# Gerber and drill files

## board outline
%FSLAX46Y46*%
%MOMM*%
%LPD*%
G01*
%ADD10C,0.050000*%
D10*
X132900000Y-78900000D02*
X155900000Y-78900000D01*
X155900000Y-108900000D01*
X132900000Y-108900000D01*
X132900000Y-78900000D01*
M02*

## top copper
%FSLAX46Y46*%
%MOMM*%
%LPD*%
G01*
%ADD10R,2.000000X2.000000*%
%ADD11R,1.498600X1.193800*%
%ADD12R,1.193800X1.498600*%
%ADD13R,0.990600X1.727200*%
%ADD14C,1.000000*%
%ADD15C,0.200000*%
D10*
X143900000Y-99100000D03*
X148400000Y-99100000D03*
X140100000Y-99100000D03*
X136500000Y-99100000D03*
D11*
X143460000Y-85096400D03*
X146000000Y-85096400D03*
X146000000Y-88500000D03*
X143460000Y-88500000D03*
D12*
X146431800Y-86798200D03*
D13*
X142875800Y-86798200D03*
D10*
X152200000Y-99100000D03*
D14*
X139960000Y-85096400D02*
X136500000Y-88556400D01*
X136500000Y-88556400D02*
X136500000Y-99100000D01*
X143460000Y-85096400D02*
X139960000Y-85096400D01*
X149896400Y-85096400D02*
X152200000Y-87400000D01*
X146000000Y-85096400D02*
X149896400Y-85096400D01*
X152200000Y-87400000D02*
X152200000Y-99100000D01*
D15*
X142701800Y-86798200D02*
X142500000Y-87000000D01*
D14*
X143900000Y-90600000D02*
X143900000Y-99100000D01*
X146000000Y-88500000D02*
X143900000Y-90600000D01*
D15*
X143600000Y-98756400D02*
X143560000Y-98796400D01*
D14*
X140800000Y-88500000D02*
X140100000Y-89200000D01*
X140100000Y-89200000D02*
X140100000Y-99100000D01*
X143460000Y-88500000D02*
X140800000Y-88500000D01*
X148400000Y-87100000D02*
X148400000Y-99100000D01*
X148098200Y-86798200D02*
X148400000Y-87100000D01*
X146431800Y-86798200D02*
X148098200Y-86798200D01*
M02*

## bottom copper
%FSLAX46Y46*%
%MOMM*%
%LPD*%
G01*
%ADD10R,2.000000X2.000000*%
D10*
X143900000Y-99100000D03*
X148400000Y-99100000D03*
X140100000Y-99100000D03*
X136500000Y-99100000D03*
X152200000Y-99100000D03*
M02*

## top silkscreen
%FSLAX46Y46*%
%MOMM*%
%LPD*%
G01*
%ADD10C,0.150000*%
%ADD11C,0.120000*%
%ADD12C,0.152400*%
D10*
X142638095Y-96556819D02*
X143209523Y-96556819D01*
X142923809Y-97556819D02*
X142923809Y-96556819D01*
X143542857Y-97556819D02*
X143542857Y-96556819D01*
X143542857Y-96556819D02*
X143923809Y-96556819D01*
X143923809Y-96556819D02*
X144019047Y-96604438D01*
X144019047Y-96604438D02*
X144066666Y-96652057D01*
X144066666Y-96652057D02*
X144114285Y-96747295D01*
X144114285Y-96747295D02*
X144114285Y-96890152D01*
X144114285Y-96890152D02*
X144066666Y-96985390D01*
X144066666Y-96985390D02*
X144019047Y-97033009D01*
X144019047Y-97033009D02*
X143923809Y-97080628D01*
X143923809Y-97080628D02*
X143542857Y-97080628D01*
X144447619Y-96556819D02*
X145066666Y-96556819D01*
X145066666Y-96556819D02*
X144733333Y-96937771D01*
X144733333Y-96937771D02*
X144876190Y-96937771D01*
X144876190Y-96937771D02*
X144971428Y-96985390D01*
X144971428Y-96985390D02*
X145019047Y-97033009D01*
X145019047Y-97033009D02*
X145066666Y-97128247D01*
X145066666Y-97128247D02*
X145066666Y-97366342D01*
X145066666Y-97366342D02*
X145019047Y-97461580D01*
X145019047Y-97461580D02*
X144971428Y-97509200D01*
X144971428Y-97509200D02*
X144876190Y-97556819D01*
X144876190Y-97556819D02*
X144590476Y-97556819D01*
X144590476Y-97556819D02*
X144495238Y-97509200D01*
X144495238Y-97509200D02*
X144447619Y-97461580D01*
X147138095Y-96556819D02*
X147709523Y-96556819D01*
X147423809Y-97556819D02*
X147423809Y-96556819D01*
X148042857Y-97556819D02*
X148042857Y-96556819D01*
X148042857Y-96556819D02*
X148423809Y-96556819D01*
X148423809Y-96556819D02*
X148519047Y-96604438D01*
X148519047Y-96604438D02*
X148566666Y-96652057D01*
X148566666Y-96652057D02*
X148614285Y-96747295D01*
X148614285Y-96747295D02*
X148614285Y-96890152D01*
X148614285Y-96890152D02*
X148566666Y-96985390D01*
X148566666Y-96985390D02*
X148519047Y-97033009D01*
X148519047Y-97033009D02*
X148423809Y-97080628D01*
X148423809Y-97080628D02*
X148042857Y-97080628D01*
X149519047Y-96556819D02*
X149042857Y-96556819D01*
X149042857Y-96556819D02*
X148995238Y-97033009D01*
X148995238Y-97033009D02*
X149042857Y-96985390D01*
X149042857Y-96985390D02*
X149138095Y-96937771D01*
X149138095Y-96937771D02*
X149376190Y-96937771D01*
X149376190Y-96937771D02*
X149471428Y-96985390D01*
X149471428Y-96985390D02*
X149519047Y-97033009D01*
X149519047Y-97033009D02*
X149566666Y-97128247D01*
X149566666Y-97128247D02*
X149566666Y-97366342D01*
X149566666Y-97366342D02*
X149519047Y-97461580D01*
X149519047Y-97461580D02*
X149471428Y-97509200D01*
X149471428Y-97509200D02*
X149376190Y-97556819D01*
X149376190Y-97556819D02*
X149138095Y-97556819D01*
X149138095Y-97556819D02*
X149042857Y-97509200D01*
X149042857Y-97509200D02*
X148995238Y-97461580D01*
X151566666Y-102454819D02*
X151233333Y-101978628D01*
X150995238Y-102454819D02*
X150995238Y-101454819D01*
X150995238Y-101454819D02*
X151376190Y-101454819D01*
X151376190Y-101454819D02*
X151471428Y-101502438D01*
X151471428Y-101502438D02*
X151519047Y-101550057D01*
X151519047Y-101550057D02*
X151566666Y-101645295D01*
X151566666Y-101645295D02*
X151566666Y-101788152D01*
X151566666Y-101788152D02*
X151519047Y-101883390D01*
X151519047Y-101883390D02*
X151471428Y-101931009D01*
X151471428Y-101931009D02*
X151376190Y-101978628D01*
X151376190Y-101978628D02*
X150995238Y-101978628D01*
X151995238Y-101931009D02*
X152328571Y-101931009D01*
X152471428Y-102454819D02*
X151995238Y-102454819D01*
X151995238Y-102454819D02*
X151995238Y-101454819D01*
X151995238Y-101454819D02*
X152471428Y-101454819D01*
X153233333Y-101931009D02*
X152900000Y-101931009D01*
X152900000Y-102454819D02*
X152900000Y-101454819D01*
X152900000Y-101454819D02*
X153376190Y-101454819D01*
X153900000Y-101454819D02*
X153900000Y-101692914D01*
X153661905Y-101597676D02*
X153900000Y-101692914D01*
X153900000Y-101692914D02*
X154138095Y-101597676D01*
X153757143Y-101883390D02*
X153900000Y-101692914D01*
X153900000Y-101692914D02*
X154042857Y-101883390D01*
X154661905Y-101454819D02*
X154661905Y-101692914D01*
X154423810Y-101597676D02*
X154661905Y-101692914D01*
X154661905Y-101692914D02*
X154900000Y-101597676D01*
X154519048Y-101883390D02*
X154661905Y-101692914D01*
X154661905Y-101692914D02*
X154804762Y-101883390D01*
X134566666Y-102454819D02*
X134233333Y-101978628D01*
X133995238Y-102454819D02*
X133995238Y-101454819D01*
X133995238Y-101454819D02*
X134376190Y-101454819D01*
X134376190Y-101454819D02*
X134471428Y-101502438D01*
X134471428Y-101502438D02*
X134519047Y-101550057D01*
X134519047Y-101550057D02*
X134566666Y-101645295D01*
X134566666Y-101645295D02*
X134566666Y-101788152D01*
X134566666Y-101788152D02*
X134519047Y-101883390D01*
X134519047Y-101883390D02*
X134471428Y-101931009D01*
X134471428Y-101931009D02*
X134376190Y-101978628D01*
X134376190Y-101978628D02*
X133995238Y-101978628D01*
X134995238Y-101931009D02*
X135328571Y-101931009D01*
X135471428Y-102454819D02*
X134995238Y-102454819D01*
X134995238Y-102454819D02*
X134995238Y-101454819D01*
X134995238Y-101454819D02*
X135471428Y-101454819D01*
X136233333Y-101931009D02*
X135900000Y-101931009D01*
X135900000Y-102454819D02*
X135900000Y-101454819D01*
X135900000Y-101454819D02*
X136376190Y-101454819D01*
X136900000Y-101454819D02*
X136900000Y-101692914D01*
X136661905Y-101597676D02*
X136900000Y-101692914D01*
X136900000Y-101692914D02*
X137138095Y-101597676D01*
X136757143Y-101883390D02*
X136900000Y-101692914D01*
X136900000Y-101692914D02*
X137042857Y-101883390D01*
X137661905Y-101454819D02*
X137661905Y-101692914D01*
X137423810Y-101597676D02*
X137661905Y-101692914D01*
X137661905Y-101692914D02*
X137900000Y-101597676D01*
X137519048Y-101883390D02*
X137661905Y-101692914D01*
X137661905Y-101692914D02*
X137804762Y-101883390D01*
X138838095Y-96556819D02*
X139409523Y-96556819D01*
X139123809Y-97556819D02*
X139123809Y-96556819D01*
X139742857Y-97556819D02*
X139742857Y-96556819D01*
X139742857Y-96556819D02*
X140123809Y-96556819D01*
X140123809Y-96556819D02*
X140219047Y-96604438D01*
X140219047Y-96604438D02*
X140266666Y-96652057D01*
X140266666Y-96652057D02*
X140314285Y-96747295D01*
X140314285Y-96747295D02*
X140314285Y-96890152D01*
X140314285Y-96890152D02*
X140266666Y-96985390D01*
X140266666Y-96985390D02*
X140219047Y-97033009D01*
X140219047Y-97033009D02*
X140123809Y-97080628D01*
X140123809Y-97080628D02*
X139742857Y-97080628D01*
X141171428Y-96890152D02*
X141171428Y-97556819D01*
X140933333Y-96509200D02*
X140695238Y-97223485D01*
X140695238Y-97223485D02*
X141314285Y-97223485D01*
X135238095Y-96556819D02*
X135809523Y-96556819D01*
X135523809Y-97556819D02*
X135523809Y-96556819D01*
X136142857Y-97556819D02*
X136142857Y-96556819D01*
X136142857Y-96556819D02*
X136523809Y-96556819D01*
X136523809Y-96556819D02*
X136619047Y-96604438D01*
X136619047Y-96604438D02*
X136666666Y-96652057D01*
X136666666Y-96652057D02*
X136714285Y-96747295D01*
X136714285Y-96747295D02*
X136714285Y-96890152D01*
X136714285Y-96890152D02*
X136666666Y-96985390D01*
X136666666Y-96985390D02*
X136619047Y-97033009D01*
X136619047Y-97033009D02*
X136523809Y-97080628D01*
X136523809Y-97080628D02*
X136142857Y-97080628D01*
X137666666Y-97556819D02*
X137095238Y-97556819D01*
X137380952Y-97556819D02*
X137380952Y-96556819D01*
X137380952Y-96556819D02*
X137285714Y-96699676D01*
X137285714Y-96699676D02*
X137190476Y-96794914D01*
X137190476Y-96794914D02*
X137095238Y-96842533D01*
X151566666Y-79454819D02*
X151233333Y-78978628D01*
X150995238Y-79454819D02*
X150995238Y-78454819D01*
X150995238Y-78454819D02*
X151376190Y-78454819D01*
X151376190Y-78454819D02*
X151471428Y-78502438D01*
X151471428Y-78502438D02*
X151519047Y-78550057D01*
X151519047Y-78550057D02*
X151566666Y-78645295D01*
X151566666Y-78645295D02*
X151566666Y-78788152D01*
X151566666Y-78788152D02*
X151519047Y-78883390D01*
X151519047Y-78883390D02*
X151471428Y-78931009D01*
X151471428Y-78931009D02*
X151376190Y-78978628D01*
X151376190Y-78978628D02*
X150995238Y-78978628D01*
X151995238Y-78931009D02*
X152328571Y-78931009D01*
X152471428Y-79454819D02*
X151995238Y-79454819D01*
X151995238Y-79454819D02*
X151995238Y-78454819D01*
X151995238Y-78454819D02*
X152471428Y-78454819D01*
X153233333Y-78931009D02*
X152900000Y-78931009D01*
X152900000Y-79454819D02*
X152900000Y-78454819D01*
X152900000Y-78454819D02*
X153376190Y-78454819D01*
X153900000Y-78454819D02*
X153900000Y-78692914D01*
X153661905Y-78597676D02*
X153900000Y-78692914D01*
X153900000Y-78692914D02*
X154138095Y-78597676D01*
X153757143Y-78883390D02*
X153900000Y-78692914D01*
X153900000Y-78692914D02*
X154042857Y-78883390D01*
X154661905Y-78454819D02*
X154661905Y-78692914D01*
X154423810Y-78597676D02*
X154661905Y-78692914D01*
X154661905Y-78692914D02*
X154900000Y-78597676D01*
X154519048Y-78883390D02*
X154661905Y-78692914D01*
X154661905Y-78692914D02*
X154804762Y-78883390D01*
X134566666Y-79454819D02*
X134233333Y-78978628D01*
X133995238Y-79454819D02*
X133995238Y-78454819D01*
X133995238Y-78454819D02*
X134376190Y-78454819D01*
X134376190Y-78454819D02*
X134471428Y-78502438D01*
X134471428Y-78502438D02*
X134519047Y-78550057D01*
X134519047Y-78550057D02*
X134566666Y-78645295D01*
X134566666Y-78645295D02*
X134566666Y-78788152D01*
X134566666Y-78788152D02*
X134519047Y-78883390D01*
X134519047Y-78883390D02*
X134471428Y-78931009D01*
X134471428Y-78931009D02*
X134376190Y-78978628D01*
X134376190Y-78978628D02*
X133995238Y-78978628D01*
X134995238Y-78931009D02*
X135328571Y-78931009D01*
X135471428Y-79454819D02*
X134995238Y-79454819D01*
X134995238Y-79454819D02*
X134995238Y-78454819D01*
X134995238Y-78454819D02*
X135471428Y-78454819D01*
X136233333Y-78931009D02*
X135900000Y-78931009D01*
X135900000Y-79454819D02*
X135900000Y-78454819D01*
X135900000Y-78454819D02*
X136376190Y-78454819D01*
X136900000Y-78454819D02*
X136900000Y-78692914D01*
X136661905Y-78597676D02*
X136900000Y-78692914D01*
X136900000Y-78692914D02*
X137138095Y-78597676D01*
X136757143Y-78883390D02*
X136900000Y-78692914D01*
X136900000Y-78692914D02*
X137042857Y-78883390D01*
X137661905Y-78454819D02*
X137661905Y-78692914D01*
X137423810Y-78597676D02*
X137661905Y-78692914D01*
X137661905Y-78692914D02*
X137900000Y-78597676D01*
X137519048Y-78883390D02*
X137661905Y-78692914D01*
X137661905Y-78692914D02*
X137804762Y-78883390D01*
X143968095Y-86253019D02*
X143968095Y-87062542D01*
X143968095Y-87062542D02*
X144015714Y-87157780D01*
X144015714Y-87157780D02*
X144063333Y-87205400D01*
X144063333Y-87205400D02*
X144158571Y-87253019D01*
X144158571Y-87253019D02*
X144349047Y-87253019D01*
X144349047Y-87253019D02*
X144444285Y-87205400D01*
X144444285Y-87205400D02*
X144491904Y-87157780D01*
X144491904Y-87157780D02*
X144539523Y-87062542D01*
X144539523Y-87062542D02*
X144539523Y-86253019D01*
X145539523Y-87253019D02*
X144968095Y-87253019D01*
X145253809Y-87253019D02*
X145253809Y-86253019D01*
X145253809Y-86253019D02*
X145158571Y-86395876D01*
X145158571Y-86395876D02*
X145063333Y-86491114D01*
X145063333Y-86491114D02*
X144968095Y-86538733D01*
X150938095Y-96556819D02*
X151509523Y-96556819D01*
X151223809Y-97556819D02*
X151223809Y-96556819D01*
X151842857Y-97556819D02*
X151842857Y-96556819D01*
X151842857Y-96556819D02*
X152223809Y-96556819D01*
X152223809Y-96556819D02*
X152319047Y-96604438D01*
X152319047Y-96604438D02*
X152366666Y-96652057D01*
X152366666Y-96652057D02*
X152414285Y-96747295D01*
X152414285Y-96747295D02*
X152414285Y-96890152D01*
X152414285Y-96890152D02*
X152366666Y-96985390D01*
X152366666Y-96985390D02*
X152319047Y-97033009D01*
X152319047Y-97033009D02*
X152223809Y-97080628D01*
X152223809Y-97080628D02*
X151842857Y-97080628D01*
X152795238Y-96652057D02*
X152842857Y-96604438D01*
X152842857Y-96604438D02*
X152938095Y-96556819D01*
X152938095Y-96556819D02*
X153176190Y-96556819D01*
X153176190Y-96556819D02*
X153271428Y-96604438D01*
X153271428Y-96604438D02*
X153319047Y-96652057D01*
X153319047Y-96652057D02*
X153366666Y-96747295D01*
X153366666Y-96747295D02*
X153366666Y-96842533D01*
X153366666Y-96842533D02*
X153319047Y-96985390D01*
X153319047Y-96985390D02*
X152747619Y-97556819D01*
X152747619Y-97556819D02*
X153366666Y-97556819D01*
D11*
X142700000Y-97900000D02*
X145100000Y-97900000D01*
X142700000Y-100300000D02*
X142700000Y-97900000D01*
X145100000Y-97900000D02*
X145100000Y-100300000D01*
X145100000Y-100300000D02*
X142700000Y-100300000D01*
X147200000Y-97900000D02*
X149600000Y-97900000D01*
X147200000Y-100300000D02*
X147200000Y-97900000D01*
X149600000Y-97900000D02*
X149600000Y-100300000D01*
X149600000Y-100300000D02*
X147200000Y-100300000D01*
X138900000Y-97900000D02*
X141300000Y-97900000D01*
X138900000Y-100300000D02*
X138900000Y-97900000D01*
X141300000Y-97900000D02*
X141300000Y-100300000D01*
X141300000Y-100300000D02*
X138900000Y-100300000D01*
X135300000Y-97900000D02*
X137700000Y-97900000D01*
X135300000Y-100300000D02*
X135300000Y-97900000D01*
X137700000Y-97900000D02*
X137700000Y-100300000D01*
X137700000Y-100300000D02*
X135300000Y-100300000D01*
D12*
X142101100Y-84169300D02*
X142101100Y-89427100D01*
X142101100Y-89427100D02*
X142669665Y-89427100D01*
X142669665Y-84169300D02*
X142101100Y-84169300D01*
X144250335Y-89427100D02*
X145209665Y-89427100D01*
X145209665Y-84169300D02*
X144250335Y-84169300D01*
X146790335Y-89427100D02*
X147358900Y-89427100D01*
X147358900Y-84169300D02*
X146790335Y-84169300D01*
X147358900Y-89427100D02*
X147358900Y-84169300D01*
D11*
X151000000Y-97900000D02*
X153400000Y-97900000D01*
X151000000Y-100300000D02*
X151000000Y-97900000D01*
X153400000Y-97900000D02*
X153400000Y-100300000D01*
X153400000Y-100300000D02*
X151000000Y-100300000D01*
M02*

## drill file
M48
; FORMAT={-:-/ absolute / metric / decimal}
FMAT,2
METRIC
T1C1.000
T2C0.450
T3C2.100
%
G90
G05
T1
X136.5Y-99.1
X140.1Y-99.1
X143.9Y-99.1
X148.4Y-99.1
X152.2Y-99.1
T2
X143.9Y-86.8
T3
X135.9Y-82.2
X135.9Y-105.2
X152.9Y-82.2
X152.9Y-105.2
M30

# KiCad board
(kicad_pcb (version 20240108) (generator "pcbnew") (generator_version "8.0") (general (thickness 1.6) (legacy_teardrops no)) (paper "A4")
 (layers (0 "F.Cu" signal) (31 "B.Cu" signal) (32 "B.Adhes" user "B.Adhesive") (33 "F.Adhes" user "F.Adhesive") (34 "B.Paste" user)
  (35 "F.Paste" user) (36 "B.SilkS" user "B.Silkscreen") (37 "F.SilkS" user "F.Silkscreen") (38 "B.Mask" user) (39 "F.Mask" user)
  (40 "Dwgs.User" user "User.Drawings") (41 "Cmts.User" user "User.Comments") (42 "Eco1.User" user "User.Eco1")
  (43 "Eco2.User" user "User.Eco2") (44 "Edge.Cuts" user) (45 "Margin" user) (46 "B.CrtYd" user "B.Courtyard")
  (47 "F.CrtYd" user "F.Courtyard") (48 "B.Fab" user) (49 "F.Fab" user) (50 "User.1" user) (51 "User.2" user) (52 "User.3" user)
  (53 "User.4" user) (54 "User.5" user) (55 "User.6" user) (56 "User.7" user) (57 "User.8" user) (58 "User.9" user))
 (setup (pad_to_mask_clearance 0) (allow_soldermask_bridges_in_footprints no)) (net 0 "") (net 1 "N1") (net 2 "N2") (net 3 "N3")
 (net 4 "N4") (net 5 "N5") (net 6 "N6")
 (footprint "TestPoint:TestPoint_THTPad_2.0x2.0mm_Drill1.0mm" (layer "F.Cu") (at 143.9 99.1)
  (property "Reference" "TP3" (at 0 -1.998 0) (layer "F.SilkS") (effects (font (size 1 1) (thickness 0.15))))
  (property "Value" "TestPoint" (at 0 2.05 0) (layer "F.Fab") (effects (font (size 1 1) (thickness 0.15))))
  (fp_line (start -1.2 -1.2) (end 1.2 -1.2) (stroke (width 0.12) (type solid)) (layer "F.SilkS"))
  (fp_line (start -1.2 1.2) (end -1.2 -1.2) (stroke (width 0.12) (type solid)) (layer "F.SilkS"))
  (fp_line (start 1.2 -1.2) (end 1.2 1.2) (stroke (width 0.12) (type solid)) (layer "F.SilkS"))
  (fp_line (start 1.2 1.2) (end -1.2 1.2) (stroke (width 0.12) (type solid)) (layer "F.SilkS"))
  (pad "1" thru_hole rect (at 0 0) (size 2 2) (drill 1) (layers "*.Cu" "*.Mask") (remove_unused_layers no) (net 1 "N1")))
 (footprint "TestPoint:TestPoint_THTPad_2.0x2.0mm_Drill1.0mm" (layer "F.Cu") (at 148.4 99.1)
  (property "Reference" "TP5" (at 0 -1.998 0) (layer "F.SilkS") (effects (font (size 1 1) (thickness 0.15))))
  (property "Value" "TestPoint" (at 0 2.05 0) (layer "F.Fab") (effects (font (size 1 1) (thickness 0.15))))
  (fp_line (start -1.2 -1.2) (end 1.2 -1.2) (stroke (width 0.12) (type solid)) (layer "F.SilkS"))
  (fp_line (start -1.2 1.2) (end -1.2 -1.2) (stroke (width 0.12) (type solid)) (layer "F.SilkS"))
  (fp_line (start 1.2 -1.2) (end 1.2 1.2) (stroke (width 0.12) (type solid)) (layer "F.SilkS"))
  (fp_line (start 1.2 1.2) (end -1.2 1.2) (stroke (width 0.12) (type solid)) (layer "F.SilkS"))
  (pad "1" thru_hole rect (at 0 0) (size 2 2) (drill 1) (layers "*.Cu" "*.Mask") (remove_unused_layers no) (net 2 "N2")))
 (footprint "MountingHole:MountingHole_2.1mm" (layer "F.Cu") (at 152.9 105.2)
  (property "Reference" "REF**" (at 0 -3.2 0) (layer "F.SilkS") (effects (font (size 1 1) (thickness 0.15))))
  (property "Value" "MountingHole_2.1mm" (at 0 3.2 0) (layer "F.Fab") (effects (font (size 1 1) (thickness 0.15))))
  (pad "" np_thru_hole circle (at 0 0) (size 2.1 2.1) (drill 2.1) (layers "*.Cu" "*.Mask")))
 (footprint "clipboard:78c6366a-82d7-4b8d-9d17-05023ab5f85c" (layer "F.Cu") (at 143.9 86.8)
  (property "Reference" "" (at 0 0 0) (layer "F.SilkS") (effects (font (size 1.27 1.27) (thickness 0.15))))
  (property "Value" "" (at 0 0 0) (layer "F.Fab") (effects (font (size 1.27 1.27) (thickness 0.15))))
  (pad "" np_thru_hole circle (at 0 0) (size 0.45 0.45) (drill 0.45) (layers "*.Mask")))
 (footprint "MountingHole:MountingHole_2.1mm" (layer "F.Cu") (at 135.9 105.2)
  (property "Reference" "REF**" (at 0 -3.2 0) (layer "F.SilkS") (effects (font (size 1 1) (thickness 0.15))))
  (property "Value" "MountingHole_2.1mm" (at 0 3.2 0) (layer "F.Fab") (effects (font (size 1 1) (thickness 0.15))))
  (pad "" np_thru_hole circle (at 0 0) (size 2.1 2.1) (drill 2.1) (layers "*.Cu" "*.Mask")))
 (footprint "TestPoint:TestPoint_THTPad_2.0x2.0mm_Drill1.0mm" (layer "F.Cu") (at 140.1 99.1)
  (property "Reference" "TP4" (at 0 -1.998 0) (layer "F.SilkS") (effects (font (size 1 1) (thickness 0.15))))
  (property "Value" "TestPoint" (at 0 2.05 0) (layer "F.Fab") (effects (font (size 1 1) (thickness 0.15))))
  (fp_line (start -1.2 -1.2) (end 1.2 -1.2) (stroke (width 0.12) (type solid)) (layer "F.SilkS"))
  (fp_line (start -1.2 1.2) (end -1.2 -1.2) (stroke (width 0.12) (type solid)) (layer "F.SilkS"))
  (fp_line (start 1.2 -1.2) (end 1.2 1.2) (stroke (width 0.12) (type solid)) (layer "F.SilkS"))
  (fp_line (start 1.2 1.2) (end -1.2 1.2) (stroke (width 0.12) (type solid)) (layer "F.SilkS"))
  (pad "1" thru_hole rect (at 0 0) (size 2 2) (drill 1) (layers "*.Cu" "*.Mask") (remove_unused_layers no) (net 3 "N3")))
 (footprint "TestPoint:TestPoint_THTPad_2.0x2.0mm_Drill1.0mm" (layer "F.Cu") (at 136.5 99.1)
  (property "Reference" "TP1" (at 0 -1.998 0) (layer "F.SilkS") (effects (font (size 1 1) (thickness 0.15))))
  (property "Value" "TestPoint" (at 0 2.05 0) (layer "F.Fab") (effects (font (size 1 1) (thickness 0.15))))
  (fp_line (start -1.2 -1.2) (end 1.2 -1.2) (stroke (width 0.12) (type solid)) (layer "F.SilkS"))
  (fp_line (start -1.2 1.2) (end -1.2 -1.2) (stroke (width 0.12) (type solid)) (layer "F.SilkS"))
  (fp_line (start 1.2 -1.2) (end 1.2 1.2) (stroke (width 0.12) (type solid)) (layer "F.SilkS"))
  (fp_line (start 1.2 1.2) (end -1.2 1.2) (stroke (width 0.12) (type solid)) (layer "F.SilkS"))
  (pad "1" thru_hole rect (at 0 0) (size 2 2) (drill 1) (layers "*.Cu" "*.Mask") (remove_unused_layers no) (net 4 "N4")))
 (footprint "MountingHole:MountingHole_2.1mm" (layer "F.Cu") (at 152.9 82.2)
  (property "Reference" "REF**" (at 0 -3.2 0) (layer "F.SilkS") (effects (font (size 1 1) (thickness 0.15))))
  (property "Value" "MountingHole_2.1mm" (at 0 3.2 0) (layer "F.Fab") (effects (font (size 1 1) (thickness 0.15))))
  (pad "" np_thru_hole circle (at 0 0) (size 2.1 2.1) (drill 2.1) (layers "*.Cu" "*.Mask")))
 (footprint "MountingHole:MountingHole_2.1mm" (layer "F.Cu") (at 135.9 82.2)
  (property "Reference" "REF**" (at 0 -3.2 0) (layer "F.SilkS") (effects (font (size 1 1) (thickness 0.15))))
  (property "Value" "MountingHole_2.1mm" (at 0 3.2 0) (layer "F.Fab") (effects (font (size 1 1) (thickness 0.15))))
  (pad "" np_thru_hole circle (at 0 0) (size 2.1 2.1) (drill 2.1) (layers "*.Cu" "*.Mask")))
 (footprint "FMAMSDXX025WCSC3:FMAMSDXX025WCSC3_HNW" (layer "F.Cu") (at 144.73 86.7982)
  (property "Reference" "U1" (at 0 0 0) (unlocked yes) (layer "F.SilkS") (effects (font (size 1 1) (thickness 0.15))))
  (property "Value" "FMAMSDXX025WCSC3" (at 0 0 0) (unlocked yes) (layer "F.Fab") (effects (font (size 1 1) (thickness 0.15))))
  (fp_line (start -2.6289 -2.6289) (end -2.6289 2.6289) (stroke (width 0.1524) (type solid)) (layer "F.SilkS"))
  (fp_line (start -2.6289 2.6289) (end -2.060335 2.6289) (stroke (width 0.1524) (type solid)) (layer "F.SilkS"))
  (fp_line (start -2.060335 -2.6289) (end -2.6289 -2.6289) (stroke (width 0.1524) (type solid)) (layer "F.SilkS"))
  (fp_line (start -0.479665 2.6289) (end 0.479665 2.6289) (stroke (width 0.1524) (type solid)) (layer "F.SilkS"))
  (fp_line (start 0.479665 -2.6289) (end -0.479665 -2.6289) (stroke (width 0.1524) (type solid)) (layer "F.SilkS"))
  (fp_line (start 2.060335 2.6289) (end 2.6289 2.6289) (stroke (width 0.1524) (type solid)) (layer "F.SilkS"))
  (fp_line (start 2.6289 -2.6289) (end 2.060335 -2.6289) (stroke (width 0.1524) (type solid)) (layer "F.SilkS"))
  (fp_line (start 2.6289 2.6289) (end 2.6289 -2.6289) (stroke (width 0.1524) (type solid)) (layer "F.SilkS"))
  (pad "1" smd rect (at -1.27 -1.7018) (size 1.4986 1.1938) (layers "F.Cu" "F.Paste" "F.Mask") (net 4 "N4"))
  (pad "2" smd rect (at 1.27 -1.7018) (size 1.4986 1.1938) (layers "F.Cu" "F.Paste" "F.Mask") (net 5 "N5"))
  (pad "3" smd rect (at 1.27 1.7018) (size 1.4986 1.1938) (layers "F.Cu" "F.Paste" "F.Mask") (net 1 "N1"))
  (pad "4" smd rect (at -1.27 1.7018) (size 1.4986 1.1938) (layers "F.Cu" "F.Paste" "F.Mask") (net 3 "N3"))
  (pad "5" smd rect (at 1.7018 0) (size 1.1938 1.4986) (layers "F.Cu" "F.Mask") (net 2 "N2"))
  (pad "6" smd rect (at -1.8542 0) (size 0.9906 1.7272) (layers "F.Cu" "F.Paste" "F.Mask") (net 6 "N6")))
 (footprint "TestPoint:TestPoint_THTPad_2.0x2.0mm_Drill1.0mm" (layer "F.Cu") (at 152.2 99.1)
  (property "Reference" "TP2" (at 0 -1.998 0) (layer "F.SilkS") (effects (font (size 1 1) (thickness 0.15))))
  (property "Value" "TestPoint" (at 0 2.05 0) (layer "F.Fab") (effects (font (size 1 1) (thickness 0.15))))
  (fp_line (start -1.2 -1.2) (end 1.2 -1.2) (stroke (width 0.12) (type solid)) (layer "F.SilkS"))
  (fp_line (start -1.2 1.2) (end -1.2 -1.2) (stroke (width 0.12) (type solid)) (layer "F.SilkS"))
  (fp_line (start 1.2 -1.2) (end 1.2 1.2) (stroke (width 0.12) (type solid)) (layer "F.SilkS"))
  (fp_line (start 1.2 1.2) (end -1.2 1.2) (stroke (width 0.12) (type solid)) (layer "F.SilkS"))
  (pad "1" thru_hole rect (at 0 0) (size 2 2) (drill 1) (layers "*.Cu" "*.Mask") (remove_unused_layers no) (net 5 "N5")))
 (gr_rect (start 132.9 78.9) (end 155.9 108.9) (stroke (width 0.05) (type default)) (fill none) (layer "Edge.Cuts"))
 (segment (start 139.96 85.0964) (end 136.5 88.5564) (width 1) (layer "F.Cu") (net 4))
 (segment (start 136.5 88.5564) (end 136.5 99.1) (width 1) (layer "F.Cu") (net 4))
 (segment (start 143.46 85.0964) (end 139.96 85.0964) (width 1) (layer "F.Cu") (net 4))
 (segment (start 149.8964 85.0964) (end 152.2 87.4) (width 1) (layer "F.Cu") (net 5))
 (segment (start 146 85.0964) (end 149.8964 85.0964) (width 1) (layer "F.Cu") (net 5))
 (segment (start 152.2 87.4) (end 152.2 99.1) (width 1) (layer "F.Cu") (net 5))
 (segment (start 142.7018 86.7982) (end 142.5 87) (width 0.2) (layer "F.Cu") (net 6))
 (segment (start 143.9 90.6) (end 143.9 99.1) (width 1) (layer "F.Cu") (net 1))
 (segment (start 146 88.5) (end 143.9 90.6) (width 1) (layer "F.Cu") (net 1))
 (segment (start 143.6 98.7564) (end 143.56 98.7964) (width 0.2) (layer "F.Cu") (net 1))
 (segment (start 140.8 88.5) (end 140.1 89.2) (width 1) (layer "F.Cu") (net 3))
 (segment (start 140.1 89.2) (end 140.1 99.1) (width 1) (layer "F.Cu") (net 3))
 (segment (start 143.46 88.5) (end 140.8 88.5) (width 1) (layer "F.Cu") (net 3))
 (segment (start 148.4 87.1) (end 148.4 99.1) (width 1) (layer "F.Cu") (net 2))
 (segment (start 148.0982 86.7982) (end 148.4 87.1) (width 1) (layer "F.Cu") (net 2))
 (segment (start 146.4318 86.7982) (end 148.0982 86.7982) (width 1) (layer "F.Cu") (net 2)))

